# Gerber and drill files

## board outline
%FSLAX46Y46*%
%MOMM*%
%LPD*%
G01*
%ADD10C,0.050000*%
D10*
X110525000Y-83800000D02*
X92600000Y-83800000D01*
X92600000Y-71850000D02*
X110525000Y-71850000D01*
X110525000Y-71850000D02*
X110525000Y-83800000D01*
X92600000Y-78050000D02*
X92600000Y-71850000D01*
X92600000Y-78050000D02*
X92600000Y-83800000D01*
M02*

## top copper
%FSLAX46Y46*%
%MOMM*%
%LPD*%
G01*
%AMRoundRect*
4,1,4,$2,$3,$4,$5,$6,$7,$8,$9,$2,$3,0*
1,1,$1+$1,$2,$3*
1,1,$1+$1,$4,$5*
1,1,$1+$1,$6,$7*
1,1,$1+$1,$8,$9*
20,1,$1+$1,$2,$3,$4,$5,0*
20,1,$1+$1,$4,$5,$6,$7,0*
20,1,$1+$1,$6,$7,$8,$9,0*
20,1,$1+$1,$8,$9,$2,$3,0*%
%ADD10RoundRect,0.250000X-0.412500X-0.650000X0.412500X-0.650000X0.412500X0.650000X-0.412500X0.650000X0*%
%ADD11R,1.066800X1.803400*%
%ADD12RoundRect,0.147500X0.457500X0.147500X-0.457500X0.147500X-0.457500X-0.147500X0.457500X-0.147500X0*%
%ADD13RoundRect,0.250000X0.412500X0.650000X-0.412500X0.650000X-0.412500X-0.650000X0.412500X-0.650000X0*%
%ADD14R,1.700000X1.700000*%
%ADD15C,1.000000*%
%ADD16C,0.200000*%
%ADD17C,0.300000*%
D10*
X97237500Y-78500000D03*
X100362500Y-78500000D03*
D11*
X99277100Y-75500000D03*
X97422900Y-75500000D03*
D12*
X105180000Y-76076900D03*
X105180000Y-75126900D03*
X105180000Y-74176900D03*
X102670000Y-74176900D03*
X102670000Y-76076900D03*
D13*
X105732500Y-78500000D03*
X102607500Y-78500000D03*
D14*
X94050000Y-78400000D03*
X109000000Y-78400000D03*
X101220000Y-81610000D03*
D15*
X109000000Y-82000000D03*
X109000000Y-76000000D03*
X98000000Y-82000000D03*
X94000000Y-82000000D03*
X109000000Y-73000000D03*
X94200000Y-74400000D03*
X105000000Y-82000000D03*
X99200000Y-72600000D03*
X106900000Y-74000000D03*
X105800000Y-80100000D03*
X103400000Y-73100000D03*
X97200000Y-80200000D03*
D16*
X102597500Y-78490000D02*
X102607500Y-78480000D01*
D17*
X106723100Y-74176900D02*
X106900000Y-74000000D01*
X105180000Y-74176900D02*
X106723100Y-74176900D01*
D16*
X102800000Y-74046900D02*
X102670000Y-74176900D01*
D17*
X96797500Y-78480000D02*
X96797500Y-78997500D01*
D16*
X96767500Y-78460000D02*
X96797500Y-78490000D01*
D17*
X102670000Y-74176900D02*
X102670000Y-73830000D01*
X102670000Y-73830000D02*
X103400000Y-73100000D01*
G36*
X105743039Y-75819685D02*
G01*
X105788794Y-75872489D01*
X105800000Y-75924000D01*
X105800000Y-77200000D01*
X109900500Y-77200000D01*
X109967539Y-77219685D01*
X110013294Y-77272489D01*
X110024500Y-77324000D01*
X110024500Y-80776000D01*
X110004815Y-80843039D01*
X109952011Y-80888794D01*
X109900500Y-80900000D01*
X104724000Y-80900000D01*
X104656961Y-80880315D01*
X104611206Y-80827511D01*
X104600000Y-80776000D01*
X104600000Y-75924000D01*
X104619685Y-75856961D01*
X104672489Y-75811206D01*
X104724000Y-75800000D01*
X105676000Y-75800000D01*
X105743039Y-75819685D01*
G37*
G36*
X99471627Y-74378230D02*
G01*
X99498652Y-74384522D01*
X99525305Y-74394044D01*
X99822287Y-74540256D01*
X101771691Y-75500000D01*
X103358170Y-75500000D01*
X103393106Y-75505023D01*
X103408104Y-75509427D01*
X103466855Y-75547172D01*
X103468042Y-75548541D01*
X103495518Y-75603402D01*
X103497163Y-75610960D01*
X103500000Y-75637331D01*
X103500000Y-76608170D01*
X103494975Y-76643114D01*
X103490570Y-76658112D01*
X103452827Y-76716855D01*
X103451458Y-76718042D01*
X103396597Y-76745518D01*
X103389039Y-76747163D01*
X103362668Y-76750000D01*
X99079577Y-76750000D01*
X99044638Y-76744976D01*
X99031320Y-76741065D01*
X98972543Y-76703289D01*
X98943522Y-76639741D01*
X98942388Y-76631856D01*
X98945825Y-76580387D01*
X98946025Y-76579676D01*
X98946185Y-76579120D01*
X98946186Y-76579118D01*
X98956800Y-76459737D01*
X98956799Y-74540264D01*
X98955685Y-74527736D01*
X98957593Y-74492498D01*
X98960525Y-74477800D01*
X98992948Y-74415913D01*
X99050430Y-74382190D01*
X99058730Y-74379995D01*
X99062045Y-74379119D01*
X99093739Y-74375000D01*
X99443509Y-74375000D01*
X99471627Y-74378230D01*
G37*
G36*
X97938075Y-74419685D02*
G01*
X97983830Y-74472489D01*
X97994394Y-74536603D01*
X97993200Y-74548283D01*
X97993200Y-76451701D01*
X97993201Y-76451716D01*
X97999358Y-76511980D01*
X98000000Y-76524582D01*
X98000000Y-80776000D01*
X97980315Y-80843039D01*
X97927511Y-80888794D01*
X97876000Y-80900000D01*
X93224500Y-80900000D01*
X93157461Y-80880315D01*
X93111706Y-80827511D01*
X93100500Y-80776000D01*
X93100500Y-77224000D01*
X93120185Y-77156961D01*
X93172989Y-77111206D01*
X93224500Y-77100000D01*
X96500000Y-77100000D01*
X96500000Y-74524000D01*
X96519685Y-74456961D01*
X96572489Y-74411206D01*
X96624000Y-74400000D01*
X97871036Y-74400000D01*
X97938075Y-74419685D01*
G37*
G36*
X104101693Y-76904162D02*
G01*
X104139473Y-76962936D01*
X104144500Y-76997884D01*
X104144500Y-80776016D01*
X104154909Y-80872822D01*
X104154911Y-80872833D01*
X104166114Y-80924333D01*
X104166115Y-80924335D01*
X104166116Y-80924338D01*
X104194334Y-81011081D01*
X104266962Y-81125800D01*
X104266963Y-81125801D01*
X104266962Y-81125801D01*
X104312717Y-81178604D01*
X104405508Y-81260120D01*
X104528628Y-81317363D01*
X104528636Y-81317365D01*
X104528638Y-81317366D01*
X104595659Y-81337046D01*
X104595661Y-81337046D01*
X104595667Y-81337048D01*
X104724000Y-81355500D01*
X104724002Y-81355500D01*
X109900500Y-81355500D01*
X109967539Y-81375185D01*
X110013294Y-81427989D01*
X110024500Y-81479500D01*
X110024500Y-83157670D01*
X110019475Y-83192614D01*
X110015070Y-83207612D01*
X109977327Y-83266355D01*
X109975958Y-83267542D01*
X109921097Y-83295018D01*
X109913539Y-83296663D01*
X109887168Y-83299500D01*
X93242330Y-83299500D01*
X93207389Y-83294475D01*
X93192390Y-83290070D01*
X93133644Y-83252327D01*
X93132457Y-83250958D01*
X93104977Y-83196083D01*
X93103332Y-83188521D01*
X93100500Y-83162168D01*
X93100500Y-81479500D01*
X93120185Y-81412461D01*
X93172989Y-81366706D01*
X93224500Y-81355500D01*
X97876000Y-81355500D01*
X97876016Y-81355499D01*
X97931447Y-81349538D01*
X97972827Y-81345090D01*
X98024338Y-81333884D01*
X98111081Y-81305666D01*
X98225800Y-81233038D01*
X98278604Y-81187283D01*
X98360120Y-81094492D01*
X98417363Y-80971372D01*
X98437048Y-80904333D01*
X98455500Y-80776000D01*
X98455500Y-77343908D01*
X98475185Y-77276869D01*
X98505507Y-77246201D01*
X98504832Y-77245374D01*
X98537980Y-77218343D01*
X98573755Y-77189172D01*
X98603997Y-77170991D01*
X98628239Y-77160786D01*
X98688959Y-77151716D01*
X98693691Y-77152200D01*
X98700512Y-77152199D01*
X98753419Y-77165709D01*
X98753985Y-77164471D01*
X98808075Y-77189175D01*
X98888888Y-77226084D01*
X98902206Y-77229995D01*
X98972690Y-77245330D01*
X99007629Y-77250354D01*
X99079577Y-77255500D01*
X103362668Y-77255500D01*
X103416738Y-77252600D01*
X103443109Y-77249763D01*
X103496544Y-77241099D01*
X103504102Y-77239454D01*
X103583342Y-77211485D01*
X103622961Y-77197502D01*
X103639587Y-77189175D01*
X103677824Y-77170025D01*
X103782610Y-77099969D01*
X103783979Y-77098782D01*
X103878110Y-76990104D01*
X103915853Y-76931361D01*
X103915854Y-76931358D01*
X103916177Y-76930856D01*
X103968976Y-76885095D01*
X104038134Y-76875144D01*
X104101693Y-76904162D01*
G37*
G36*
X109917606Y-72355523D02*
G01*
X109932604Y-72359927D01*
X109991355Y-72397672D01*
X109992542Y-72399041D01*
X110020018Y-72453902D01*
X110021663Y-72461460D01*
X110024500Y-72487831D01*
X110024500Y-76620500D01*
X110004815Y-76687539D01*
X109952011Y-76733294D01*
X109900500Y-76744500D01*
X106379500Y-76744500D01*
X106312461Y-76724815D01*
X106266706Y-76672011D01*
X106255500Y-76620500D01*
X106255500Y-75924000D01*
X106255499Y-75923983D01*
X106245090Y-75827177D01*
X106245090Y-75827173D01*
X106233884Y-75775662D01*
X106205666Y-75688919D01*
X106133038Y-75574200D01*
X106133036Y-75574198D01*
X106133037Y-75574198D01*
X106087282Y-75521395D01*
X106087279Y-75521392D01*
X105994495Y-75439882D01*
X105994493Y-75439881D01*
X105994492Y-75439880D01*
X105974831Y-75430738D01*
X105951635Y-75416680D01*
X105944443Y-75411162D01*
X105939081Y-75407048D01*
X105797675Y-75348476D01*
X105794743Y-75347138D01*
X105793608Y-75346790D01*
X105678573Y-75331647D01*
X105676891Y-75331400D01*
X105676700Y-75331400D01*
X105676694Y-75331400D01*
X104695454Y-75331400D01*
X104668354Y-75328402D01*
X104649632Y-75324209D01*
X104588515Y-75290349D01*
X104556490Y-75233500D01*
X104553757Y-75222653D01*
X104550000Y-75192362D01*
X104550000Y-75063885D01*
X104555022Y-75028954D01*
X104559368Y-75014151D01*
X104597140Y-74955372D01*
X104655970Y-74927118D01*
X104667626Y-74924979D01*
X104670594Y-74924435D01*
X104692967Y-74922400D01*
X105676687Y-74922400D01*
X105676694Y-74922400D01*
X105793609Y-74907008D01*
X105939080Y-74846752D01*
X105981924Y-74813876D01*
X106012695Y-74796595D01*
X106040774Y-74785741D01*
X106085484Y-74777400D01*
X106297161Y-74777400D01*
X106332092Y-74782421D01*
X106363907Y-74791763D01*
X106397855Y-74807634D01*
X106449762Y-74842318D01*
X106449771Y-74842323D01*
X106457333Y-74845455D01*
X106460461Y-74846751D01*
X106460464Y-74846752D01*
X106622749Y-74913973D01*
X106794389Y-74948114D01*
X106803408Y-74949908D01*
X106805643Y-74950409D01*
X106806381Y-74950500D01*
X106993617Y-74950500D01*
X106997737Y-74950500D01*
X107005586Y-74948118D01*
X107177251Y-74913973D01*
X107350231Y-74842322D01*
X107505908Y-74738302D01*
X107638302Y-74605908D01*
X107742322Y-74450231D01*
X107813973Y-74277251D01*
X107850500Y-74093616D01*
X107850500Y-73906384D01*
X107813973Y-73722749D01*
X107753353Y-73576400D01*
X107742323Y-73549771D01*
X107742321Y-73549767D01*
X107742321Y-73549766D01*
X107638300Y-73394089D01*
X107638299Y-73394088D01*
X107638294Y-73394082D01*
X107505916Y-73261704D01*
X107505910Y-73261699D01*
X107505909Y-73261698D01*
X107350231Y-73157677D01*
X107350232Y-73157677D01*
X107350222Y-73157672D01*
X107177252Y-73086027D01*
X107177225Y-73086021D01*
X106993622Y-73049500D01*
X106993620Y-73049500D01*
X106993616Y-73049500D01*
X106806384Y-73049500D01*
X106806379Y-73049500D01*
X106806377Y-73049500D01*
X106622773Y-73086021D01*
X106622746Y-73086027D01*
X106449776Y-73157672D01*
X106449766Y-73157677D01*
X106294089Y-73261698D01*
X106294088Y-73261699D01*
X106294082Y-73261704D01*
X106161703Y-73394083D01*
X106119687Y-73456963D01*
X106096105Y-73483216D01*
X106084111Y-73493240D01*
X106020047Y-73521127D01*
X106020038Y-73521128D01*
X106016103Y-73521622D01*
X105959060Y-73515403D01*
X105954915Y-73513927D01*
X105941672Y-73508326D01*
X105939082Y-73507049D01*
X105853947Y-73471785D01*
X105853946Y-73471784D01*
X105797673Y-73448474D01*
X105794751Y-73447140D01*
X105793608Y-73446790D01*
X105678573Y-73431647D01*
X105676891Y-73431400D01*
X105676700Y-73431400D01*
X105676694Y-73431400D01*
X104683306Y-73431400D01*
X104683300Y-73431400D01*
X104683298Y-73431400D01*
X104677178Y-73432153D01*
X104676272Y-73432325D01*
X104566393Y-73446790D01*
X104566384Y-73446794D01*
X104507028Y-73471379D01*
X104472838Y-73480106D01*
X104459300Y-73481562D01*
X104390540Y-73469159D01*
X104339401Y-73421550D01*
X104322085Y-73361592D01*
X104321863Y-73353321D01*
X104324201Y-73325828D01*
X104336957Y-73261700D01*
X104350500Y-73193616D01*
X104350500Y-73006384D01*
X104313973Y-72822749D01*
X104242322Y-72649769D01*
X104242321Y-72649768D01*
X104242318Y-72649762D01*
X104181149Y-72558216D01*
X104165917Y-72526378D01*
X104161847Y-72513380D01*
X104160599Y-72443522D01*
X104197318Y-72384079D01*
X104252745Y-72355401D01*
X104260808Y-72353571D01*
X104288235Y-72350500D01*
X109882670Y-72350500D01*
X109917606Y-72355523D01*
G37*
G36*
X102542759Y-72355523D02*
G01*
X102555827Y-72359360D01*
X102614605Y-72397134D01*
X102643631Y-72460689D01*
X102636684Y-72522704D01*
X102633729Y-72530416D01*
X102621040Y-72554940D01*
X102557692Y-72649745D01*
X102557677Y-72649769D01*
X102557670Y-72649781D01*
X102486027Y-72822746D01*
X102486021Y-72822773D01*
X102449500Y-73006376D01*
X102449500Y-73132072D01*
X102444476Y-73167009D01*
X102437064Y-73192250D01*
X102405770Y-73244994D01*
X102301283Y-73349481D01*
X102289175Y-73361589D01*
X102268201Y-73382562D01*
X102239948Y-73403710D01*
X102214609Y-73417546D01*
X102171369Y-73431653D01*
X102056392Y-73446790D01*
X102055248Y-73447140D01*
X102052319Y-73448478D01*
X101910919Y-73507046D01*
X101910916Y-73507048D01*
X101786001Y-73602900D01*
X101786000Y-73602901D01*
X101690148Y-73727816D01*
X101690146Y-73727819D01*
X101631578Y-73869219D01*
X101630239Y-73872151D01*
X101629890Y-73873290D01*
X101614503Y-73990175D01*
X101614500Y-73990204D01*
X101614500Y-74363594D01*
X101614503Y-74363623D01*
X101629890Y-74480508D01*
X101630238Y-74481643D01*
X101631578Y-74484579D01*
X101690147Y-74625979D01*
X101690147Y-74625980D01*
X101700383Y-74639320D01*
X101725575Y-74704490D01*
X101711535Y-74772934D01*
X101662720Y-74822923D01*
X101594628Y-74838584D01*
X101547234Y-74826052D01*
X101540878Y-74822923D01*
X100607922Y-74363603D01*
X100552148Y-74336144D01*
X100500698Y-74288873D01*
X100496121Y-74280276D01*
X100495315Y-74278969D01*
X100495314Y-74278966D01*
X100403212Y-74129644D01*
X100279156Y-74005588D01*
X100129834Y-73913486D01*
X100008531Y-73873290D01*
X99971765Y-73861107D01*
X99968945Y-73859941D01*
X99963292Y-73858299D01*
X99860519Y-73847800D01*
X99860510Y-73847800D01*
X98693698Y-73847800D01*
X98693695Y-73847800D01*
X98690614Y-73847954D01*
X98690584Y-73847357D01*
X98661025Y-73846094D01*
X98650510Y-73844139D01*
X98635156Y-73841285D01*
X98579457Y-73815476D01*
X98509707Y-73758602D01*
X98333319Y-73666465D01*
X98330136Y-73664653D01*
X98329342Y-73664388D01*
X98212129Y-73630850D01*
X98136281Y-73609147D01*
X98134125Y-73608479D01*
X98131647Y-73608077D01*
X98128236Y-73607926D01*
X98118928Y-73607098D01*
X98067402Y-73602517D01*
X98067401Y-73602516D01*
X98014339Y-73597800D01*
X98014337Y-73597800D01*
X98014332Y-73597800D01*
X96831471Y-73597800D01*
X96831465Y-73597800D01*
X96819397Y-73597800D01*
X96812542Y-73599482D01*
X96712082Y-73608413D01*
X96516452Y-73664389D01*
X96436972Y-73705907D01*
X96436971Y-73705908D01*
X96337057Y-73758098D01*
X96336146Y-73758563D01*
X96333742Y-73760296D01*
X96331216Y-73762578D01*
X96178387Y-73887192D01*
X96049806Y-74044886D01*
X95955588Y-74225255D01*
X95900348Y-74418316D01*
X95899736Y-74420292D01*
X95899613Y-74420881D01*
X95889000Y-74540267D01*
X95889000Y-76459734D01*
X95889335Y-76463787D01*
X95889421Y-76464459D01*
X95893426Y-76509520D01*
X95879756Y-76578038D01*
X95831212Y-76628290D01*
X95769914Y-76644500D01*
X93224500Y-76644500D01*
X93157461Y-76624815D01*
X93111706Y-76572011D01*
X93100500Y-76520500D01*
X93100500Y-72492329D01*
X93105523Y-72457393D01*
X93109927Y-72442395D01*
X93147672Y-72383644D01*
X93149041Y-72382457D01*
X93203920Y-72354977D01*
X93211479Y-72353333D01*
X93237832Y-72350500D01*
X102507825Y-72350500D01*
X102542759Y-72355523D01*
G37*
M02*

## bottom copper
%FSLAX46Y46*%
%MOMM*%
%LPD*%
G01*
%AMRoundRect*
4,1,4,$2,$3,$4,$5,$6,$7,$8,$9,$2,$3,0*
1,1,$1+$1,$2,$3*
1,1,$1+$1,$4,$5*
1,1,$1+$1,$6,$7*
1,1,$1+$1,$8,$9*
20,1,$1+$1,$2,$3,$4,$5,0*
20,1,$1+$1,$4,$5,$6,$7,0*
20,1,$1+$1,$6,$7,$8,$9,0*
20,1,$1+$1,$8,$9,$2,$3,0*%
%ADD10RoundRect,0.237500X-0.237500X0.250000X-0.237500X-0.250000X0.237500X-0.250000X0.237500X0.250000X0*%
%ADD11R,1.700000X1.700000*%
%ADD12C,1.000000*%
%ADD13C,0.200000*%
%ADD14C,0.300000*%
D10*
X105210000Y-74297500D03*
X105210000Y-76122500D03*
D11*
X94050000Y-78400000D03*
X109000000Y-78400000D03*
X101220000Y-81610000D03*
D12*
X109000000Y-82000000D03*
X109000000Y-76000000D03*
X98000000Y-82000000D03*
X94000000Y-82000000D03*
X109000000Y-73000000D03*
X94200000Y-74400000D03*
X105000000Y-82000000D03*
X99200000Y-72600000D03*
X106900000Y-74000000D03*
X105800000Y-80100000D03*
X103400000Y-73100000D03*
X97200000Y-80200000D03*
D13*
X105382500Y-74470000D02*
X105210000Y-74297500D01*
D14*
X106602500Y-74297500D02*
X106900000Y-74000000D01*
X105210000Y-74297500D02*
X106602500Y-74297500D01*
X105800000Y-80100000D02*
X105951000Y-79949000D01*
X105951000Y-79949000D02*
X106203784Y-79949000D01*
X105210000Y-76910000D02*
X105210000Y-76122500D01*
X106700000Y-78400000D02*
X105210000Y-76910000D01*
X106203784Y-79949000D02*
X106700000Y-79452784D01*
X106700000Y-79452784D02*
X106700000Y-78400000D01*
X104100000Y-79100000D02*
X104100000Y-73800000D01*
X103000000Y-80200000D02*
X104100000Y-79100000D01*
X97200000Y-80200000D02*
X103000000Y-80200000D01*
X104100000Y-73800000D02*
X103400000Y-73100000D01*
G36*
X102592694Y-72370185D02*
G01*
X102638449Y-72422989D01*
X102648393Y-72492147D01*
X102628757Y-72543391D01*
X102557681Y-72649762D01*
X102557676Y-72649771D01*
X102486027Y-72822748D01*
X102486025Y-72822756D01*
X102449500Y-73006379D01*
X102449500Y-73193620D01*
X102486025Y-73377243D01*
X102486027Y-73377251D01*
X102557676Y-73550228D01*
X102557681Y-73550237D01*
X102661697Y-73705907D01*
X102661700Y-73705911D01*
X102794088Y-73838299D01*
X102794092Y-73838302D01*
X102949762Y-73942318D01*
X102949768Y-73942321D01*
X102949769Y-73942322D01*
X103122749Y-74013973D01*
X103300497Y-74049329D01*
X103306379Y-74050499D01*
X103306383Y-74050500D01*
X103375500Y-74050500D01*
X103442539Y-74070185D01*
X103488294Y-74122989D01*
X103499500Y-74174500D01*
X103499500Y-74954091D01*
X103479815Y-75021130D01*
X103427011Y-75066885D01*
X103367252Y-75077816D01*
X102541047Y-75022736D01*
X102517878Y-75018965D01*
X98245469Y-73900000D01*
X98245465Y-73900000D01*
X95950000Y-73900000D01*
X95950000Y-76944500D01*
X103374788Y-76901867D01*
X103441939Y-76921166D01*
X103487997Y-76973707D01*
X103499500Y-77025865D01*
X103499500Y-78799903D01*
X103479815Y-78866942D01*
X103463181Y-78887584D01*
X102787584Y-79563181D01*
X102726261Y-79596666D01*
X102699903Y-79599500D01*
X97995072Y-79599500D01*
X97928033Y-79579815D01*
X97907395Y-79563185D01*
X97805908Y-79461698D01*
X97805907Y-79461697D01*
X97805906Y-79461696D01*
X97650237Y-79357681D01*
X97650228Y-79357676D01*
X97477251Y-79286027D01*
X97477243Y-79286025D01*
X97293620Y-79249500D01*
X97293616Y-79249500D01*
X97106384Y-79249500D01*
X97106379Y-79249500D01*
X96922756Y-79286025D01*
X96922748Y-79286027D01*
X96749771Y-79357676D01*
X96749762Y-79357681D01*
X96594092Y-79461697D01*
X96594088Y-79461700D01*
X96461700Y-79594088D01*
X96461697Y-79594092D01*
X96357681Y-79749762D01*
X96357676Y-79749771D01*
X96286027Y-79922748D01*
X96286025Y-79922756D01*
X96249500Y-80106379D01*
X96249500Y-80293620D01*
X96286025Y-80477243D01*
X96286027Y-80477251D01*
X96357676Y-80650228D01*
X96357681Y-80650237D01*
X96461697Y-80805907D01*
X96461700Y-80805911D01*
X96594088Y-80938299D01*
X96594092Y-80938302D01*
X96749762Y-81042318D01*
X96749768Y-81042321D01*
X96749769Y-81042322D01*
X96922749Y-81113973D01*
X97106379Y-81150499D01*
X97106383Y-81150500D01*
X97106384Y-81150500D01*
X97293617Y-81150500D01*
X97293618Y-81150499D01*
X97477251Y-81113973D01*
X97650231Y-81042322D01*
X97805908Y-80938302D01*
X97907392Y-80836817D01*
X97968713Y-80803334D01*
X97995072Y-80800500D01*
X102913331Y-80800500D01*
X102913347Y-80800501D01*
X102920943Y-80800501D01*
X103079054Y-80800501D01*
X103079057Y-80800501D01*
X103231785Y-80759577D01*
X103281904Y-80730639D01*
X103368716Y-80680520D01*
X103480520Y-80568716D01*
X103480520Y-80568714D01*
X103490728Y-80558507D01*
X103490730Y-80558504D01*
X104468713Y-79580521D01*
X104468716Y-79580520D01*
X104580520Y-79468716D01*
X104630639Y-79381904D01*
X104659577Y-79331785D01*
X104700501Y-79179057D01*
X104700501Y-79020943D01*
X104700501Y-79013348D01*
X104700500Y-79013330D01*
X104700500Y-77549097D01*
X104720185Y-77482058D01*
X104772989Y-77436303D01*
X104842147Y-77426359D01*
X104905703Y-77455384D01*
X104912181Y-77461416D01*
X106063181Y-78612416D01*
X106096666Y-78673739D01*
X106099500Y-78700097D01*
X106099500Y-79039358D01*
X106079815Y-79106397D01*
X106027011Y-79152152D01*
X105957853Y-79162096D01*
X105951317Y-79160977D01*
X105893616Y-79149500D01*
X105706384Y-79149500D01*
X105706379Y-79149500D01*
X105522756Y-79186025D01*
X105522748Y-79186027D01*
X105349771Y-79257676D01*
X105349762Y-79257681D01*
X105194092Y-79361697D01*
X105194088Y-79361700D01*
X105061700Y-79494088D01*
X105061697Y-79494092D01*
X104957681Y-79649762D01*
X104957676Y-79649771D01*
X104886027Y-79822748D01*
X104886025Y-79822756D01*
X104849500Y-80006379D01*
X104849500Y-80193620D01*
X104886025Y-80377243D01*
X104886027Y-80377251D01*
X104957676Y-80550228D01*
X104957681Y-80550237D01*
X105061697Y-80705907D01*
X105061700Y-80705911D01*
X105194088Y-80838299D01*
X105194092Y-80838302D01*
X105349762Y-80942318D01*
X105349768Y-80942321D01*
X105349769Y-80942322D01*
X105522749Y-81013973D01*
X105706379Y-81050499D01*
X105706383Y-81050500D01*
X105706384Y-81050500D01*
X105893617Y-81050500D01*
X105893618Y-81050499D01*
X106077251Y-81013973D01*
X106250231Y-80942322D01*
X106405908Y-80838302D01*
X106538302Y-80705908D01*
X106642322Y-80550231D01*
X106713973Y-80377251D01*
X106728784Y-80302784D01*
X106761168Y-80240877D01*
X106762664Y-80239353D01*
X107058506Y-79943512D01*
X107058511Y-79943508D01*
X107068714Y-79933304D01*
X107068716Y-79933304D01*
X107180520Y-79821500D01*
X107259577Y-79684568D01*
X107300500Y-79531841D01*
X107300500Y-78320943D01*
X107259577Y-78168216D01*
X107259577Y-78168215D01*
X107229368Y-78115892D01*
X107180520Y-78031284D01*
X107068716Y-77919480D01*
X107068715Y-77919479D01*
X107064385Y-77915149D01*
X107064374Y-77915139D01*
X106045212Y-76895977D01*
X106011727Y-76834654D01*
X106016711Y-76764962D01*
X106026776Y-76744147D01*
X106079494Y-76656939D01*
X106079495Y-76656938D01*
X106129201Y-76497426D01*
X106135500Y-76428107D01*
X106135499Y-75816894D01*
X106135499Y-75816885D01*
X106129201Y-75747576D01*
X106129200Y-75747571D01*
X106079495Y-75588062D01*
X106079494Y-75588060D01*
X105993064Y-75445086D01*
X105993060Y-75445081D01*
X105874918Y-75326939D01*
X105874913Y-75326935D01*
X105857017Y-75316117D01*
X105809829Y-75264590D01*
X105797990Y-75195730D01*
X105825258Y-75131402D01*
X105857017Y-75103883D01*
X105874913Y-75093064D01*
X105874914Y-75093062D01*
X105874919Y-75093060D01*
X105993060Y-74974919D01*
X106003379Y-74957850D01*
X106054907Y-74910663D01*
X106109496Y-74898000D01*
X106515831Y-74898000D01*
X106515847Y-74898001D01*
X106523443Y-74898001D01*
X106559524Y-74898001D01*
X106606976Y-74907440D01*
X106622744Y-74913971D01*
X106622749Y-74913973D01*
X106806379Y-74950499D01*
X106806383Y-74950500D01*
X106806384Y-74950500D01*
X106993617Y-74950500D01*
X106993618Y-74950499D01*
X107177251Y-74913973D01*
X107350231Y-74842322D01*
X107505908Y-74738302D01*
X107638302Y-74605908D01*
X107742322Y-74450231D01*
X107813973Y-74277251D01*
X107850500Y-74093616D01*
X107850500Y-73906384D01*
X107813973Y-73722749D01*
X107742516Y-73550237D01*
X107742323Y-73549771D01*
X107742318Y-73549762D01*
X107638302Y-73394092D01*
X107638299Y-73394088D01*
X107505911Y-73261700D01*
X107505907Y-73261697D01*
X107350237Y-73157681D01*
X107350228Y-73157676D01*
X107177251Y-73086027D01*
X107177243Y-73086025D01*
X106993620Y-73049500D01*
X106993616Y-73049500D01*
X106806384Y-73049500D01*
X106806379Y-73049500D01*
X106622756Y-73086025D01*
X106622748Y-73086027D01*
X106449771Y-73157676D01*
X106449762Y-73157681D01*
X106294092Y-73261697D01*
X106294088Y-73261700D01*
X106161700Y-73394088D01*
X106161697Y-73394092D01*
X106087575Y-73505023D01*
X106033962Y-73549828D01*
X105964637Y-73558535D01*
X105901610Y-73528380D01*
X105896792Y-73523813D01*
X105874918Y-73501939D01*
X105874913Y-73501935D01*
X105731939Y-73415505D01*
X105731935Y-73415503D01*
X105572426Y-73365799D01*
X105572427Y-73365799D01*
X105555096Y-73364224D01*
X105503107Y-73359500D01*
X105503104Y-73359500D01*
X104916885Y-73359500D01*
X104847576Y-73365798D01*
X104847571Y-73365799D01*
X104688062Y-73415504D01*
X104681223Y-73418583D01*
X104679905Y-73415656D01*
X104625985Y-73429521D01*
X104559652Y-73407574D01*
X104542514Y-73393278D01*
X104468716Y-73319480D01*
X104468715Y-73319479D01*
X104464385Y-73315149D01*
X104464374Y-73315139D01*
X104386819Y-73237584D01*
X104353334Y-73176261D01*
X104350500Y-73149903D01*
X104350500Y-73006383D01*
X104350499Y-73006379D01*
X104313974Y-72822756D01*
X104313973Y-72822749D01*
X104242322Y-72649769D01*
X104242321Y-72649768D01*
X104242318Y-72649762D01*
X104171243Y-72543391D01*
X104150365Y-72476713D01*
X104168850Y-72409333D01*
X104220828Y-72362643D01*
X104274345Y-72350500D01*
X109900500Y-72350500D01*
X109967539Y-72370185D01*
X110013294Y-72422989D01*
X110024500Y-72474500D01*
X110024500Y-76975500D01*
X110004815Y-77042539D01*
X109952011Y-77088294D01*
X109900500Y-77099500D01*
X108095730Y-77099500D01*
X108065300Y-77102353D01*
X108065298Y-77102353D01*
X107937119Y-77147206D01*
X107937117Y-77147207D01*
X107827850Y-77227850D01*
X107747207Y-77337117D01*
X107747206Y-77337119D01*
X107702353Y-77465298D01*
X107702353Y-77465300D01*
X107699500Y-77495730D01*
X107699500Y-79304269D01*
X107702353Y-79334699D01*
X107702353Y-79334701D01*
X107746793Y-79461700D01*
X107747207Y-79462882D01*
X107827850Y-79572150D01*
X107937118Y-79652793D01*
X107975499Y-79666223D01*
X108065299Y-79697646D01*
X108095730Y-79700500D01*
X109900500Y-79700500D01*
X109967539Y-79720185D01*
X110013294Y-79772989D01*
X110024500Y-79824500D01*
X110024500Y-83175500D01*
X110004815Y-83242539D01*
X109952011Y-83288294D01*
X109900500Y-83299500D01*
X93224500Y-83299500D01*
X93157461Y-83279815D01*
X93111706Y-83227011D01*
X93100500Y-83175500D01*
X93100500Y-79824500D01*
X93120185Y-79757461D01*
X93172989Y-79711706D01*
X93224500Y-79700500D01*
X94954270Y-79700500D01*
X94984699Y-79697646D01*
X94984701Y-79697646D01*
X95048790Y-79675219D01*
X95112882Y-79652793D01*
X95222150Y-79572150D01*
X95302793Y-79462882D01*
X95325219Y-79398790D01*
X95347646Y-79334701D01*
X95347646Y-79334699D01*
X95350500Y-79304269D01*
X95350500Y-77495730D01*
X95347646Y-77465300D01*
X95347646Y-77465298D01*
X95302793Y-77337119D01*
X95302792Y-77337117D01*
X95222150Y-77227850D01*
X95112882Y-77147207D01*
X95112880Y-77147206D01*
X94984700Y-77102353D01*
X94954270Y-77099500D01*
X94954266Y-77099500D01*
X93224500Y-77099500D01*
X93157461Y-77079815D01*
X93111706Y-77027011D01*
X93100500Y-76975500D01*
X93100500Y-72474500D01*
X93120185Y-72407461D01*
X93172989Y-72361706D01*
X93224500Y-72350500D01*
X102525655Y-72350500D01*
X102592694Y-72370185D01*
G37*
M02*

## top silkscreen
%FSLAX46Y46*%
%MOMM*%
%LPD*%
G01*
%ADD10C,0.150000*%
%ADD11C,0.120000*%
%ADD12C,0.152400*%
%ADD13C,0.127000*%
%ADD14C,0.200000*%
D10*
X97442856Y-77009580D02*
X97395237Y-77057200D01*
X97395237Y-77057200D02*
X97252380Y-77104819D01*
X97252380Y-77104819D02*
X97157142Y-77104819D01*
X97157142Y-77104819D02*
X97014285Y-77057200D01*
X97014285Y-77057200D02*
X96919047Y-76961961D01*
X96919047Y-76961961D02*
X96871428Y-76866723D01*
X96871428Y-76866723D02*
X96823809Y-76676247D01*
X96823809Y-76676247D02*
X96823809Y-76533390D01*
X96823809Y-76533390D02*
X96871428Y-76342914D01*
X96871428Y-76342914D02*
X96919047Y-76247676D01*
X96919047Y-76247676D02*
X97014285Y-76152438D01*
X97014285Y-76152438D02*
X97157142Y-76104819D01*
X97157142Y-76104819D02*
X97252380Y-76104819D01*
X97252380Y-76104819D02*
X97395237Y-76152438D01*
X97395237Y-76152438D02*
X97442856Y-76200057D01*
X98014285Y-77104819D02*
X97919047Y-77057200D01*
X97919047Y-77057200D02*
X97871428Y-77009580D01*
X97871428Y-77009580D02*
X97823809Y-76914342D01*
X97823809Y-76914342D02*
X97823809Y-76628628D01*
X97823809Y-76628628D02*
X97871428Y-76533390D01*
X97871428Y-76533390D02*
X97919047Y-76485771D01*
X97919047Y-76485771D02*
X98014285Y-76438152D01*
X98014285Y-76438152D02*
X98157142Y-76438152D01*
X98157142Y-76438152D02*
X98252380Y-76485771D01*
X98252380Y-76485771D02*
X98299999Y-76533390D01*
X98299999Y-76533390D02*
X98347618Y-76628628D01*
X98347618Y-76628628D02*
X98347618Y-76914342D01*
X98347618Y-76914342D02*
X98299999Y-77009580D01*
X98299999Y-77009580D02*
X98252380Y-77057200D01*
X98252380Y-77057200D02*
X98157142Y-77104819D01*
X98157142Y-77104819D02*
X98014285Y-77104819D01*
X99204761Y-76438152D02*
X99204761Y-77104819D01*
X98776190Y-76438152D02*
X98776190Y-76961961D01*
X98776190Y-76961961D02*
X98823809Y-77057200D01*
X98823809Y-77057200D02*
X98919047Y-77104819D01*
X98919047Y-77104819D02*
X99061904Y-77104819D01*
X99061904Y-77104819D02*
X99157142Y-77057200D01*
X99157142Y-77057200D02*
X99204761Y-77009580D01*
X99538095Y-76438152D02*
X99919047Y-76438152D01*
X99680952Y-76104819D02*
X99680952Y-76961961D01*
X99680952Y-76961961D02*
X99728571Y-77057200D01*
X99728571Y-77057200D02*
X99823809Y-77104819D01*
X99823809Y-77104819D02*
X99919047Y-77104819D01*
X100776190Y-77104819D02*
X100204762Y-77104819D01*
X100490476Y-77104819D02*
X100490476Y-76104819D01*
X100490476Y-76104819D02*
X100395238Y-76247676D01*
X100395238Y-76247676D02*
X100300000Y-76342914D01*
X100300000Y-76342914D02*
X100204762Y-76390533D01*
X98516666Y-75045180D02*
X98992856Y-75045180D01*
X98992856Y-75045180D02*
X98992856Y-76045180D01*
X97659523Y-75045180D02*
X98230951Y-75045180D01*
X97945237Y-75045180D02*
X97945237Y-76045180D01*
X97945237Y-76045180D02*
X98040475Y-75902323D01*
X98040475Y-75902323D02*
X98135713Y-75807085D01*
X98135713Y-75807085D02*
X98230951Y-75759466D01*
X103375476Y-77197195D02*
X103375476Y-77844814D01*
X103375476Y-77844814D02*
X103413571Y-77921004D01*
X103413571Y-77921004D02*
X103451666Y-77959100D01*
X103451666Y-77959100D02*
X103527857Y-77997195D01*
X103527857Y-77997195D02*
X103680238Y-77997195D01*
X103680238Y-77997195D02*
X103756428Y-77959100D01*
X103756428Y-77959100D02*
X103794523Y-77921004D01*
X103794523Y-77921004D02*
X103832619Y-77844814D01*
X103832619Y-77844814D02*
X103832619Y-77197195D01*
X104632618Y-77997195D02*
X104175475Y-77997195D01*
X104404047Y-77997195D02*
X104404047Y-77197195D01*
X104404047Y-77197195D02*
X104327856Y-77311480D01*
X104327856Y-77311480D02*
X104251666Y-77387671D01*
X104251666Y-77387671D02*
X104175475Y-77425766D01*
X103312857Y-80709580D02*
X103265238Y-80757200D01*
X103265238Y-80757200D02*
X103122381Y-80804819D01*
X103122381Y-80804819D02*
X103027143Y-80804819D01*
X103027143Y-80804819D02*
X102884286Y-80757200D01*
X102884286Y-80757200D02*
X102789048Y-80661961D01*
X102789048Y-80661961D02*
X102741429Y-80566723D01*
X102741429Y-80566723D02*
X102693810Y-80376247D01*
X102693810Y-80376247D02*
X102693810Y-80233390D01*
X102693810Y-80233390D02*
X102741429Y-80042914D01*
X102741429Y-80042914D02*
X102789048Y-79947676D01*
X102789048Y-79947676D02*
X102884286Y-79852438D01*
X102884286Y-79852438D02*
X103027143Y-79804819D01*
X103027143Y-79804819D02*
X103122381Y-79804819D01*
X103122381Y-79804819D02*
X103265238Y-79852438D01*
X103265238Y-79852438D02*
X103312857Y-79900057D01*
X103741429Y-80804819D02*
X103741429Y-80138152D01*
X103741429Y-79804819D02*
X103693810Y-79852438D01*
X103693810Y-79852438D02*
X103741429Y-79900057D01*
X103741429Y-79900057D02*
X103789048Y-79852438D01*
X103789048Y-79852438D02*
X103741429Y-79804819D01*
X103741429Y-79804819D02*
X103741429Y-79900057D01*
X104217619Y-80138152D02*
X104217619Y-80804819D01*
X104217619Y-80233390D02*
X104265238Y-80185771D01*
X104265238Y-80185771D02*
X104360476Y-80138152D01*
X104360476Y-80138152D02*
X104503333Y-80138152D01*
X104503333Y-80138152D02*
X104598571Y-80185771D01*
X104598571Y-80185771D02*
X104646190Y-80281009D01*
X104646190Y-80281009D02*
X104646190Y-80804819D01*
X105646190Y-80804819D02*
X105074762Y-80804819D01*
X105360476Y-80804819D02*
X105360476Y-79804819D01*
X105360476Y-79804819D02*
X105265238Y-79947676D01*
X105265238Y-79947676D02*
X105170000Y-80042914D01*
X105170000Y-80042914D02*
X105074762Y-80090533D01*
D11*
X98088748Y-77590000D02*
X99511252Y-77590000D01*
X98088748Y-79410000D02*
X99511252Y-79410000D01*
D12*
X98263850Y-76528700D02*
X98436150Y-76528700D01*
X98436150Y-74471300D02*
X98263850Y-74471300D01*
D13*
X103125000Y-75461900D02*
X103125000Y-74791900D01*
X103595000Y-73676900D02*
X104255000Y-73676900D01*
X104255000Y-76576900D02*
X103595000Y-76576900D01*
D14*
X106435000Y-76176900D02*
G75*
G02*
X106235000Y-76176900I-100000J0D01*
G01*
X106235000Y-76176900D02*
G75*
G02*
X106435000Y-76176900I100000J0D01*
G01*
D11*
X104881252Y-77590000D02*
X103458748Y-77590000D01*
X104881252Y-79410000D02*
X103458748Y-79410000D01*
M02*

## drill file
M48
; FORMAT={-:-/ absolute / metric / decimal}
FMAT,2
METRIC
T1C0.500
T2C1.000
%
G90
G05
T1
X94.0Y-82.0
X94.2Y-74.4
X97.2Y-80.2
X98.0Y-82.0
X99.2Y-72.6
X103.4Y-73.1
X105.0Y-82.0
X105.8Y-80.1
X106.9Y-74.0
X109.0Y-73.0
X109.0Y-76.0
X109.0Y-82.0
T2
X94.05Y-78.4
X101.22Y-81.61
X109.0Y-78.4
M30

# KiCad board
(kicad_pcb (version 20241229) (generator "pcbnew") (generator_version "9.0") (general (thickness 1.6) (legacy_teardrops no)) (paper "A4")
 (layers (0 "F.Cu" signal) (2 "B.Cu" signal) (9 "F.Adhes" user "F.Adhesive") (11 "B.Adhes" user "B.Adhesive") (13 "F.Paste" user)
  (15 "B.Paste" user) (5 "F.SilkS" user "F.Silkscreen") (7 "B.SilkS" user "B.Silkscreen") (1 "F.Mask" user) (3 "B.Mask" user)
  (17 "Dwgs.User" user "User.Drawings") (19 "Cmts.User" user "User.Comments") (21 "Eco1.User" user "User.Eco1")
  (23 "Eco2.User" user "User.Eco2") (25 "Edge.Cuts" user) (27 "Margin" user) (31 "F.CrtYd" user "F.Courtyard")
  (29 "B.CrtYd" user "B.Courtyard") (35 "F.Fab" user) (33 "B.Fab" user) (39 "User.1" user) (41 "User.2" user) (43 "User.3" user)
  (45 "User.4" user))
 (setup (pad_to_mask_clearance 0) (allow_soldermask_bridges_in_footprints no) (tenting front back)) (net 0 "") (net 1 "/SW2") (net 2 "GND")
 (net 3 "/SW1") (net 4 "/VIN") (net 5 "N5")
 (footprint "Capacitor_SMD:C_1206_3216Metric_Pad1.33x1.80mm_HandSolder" (layer "F.Cu") (at 98.8 78.5)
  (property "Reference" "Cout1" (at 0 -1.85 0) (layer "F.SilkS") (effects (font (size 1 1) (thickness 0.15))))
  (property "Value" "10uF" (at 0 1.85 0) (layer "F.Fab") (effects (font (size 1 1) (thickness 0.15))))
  (fp_line (start -0.711252 -0.91) (end 0.711252 -0.91) (stroke (width 0.12) (type solid)) (layer "F.SilkS"))
  (fp_line (start -0.711252 0.91) (end 0.711252 0.91) (stroke (width 0.12) (type solid)) (layer "F.SilkS"))
  (pad "1" smd roundrect (at -1.5625 0) (size 1.325 1.8) (layers "F.Cu" "F.Mask" "F.Paste") (roundrect_rratio 0.188679) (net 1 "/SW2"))
  (pad "2" smd roundrect (at 1.5625 0) (size 1.325 1.8) (layers "F.Cu" "F.Mask" "F.Paste") (roundrect_rratio 0.188679) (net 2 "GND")))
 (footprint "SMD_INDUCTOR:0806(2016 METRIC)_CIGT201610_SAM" (layer "F.Cu") (at 98.35 75.5 180)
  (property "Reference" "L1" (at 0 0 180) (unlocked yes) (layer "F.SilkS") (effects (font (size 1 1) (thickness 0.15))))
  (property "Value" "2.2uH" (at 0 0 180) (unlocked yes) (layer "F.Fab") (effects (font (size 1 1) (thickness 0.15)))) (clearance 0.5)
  (fp_line (start 0.08615 -1.0287) (end -0.08615 -1.0287) (stroke (width 0.1524) (type solid)) (layer "F.SilkS"))
  (fp_line (start -0.08615 1.0287) (end 0.08615 1.0287) (stroke (width 0.1524) (type solid)) (layer "F.SilkS"))
  (pad "1" smd rect (at -0.9271 0 180) (size 1.0668 1.8034) (layers "F.Cu" "F.Mask" "F.Paste") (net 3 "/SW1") (clearance 0.75))
  (pad "2" smd rect (at 0.9271 0 180) (size 1.0668 1.8034) (layers "F.Cu" "F.Mask" "F.Paste") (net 1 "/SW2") (clearance 1))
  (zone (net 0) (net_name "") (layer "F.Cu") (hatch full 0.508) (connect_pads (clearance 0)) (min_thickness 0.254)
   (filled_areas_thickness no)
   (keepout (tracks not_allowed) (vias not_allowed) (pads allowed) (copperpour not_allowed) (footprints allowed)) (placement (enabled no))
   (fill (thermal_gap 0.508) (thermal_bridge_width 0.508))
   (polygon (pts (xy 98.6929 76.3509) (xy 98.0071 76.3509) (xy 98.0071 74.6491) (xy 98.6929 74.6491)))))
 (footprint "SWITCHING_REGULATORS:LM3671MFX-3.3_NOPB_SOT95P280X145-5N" (layer "F.Cu") (at 103.925 75.1269 180)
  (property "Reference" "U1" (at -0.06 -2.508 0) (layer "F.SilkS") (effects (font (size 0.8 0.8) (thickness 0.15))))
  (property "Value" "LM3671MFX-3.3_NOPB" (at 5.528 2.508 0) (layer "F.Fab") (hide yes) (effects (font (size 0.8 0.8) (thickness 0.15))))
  (fp_line (start 0.8 -0.335) (end 0.8 0.335) (stroke (width 0.127) (type solid)) (layer "F.SilkS"))
  (fp_line (start 0.33 1.45) (end -0.33 1.45) (stroke (width 0.127) (type solid)) (layer "F.SilkS"))
  (fp_line (start -0.33 -1.45) (end 0.33 -1.45) (stroke (width 0.127) (type solid)) (layer "F.SilkS"))
  (fp_circle (center -2.41 -1.05) (end -2.31 -1.05) (stroke (width 0.2) (type solid)) (fill no) (layer "F.SilkS"))
  (pad "1" smd roundrect (at -1.255 -0.95 180) (size 1.21 0.59) (layers "F.Cu" "F.Mask" "F.Paste") (roundrect_rratio 0.25) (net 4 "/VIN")
   (solder_mask_margin 0.102))
  (pad "2" smd roundrect (at -1.255 0 180) (size 1.21 0.59) (layers "F.Cu" "F.Mask" "F.Paste") (roundrect_rratio 0.25) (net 2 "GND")
   (solder_mask_margin 0.102))
  (pad "3" smd roundrect (at -1.255 0.95 180) (size 1.21 0.59) (layers "F.Cu" "F.Mask" "F.Paste") (roundrect_rratio 0.25) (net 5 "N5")
   (solder_mask_margin 0.102))
  (pad "4" smd roundrect (at 1.255 0.95 180) (size 1.21 0.59) (layers "F.Cu" "F.Mask" "F.Paste") (roundrect_rratio 0.25) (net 1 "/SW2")
   (solder_mask_margin 0.102))
  (pad "5" smd roundrect (at 1.255 -0.95 180) (size 1.21 0.59) (layers "F.Cu" "F.Mask" "F.Paste") (roundrect_rratio 0.25) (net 3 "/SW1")
   (solder_mask_margin 0.102)))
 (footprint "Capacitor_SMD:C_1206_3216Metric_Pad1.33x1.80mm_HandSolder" (layer "F.Cu") (at 104.17 78.5 180)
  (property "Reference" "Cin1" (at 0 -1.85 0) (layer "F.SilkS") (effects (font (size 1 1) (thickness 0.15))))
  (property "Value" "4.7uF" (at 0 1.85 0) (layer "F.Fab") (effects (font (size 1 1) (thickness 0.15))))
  (fp_line (start -0.711252 0.91) (end 0.711252 0.91) (stroke (width 0.12) (type solid)) (layer "F.SilkS"))
  (fp_line (start -0.711252 -0.91) (end 0.711252 -0.91) (stroke (width 0.12) (type solid)) (layer "F.SilkS"))
  (pad "1" smd roundrect (at -1.5625 0 180) (size 1.325 1.8) (layers "F.Cu" "F.Mask" "F.Paste") (roundrect_rratio 0.188679) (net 4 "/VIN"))
  (pad "2" smd roundrect (at 1.5625 0 180) (size 1.325 1.8) (layers "F.Cu" "F.Mask" "F.Paste") (roundrect_rratio 0.188679) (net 2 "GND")))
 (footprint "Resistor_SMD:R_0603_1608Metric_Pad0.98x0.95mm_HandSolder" (layer "B.Cu") (at 105.21 75.21 -90)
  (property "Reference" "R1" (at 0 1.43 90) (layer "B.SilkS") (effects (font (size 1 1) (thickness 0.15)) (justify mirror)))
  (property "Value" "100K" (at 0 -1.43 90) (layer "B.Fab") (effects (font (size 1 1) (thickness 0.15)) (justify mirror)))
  (pad "1" smd roundrect (at -0.9125 0 270) (size 0.975 0.95) (layers "B.Cu" "B.Mask" "B.Paste") (roundrect_rratio 0.25) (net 5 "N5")
   (clearance 0.45))
  (pad "2" smd roundrect (at 0.9125 0 270) (size 0.975 0.95) (layers "B.Cu" "B.Mask" "B.Paste") (roundrect_rratio 0.25) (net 4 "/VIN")
   (clearance 0.45)))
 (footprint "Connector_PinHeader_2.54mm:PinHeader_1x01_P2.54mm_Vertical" (layer "B.Cu") (at 94.05 78.4 180)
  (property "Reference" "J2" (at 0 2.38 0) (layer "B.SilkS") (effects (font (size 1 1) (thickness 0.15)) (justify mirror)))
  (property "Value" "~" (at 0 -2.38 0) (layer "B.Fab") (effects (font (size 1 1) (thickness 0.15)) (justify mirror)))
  (pad "3" thru_hole rect (at 0 0 180) (size 1.7 1.7) (drill 1) (layers "*.Cu" "*.Mask") (remove_unused_layers no) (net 1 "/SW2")))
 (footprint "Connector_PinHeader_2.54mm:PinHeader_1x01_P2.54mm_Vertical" (layer "B.Cu") (at 109 78.4 180)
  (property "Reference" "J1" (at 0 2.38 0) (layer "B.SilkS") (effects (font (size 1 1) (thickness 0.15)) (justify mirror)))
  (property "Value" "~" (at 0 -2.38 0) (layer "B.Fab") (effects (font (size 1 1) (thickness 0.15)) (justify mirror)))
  (pad "1" thru_hole rect (at 0 0 180) (size 1.7 1.7) (drill 1) (layers "*.Cu" "*.Mask") (remove_unused_layers no) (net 4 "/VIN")))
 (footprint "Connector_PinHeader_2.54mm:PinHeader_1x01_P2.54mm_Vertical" (layer "B.Cu") (at 101.22 81.61 180)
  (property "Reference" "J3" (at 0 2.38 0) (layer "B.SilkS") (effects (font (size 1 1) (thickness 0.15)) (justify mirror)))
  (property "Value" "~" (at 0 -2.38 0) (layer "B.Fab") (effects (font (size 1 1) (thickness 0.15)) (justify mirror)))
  (pad "2" thru_hole rect (at 0 0 180) (size 1.7 1.7) (drill 1) (layers "*.Cu" "*.Mask") (remove_unused_layers no) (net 2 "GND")))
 (gr_line (start 110.525 83.8) (end 92.6 83.8) (stroke (width 0.05) (type default)) (layer "Edge.Cuts"))
 (gr_line (start 92.6 71.85) (end 110.525 71.85) (stroke (width 0.05) (type default)) (layer "Edge.Cuts"))
 (gr_line (start 110.525 71.85) (end 110.525 83.8) (stroke (width 0.05) (type default)) (layer "Edge.Cuts"))
 (gr_line (start 92.6 78.05) (end 92.6 71.85) (stroke (width 0.05) (type default)) (layer "Edge.Cuts"))
 (gr_line (start 92.6 78.05) (end 92.6 83.8) (stroke (width 0.05) (type default)) (layer "Edge.Cuts"))
 (segment (start 102.5975 78.49) (end 102.6075 78.48) (width 0.2) (layer "F.Cu") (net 2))
 (via (at 109 82) (size 1) (drill 0.5) (layers "F.Cu" "B.Cu") (free yes) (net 2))
 (via (at 109 76) (size 1) (drill 0.5) (layers "F.Cu" "B.Cu") (free yes) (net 2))
 (via (at 98 82) (size 1) (drill 0.5) (layers "F.Cu" "B.Cu") (free yes) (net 2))
 (via (at 94 82) (size 1) (drill 0.5) (layers "F.Cu" "B.Cu") (free yes) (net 2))
 (via (at 109 73) (size 1) (drill 0.5) (layers "F.Cu" "B.Cu") (free yes) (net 2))
 (via (at 94.2 74.4) (size 1) (drill 0.5) (layers "F.Cu" "B.Cu") (free yes) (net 2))
 (via (at 105 82) (size 1) (drill 0.5) (layers "F.Cu" "B.Cu") (free yes) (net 2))
 (via (at 99.2 72.6) (size 1) (drill 0.5) (layers "F.Cu" "B.Cu") (free yes) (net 2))
 (segment (start 106.7231 74.1769) (end 106.9 74) (width 0.3) (layer "F.Cu") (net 5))
 (segment (start 105.18 74.1769) (end 106.7231 74.1769) (width 0.3) (layer "F.Cu") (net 5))
 (via (at 106.9 74) (size 1) (drill 0.5) (layers "F.Cu" "B.Cu") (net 5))
 (segment (start 105.3825 74.47) (end 105.21 74.2975) (width 0.2) (layer "B.Cu") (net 5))
 (segment (start 106.6025 74.2975) (end 106.9 74) (width 0.3) (layer "B.Cu") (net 5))
 (segment (start 105.21 74.2975) (end 106.6025 74.2975) (width 0.3) (layer "B.Cu") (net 5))
 (via (at 105.8 80.1) (size 1) (drill 0.5) (layers "F.Cu" "B.Cu") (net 4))
 (segment (start 105.8 80.1) (end 105.951 79.949) (width 0.3) (layer "B.Cu") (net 4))
 (segment (start 105.951 79.949) (end 106.203784 79.949) (width 0.3) (layer "B.Cu") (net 4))
 (segment (start 105.21 76.91) (end 105.21 76.1225) (width 0.3) (layer "B.Cu") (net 4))
 (segment (start 106.7 78.4) (end 105.21 76.91) (width 0.3) (layer "B.Cu") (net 4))
 (segment (start 106.203784 79.949) (end 106.7 79.452784) (width 0.3) (layer "B.Cu") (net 4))
 (segment (start 106.7 79.452784) (end 106.7 78.4) (width 0.3) (layer "B.Cu") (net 4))
 (segment (start 102.8 74.0469) (end 102.67 74.1769) (width 0.2) (layer "F.Cu") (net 1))
 (segment (start 96.7975 78.48) (end 96.7975 78.9975) (width 0.3) (layer "F.Cu") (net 1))
 (segment (start 96.7675 78.46) (end 96.7975 78.49) (width 0.2) (layer "F.Cu") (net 1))
 (segment (start 102.67 74.1769) (end 102.67 73.83) (width 0.3) (layer "F.Cu") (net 1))
 (segment (start 102.67 73.83) (end 103.4 73.1) (width 0.3) (layer "F.Cu") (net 1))
 (via (at 103.4 73.1) (size 1) (drill 0.5) (layers "F.Cu" "B.Cu") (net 1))
 (via (at 97.2 80.2) (size 1) (drill 0.5) (layers "F.Cu" "B.Cu") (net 1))
 (segment (start 104.1 79.1) (end 104.1 73.8) (width 0.3) (layer "B.Cu") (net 1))
 (segment (start 103 80.2) (end 104.1 79.1) (width 0.3) (layer "B.Cu") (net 1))
 (segment (start 97.2 80.2) (end 103 80.2) (width 0.3) (layer "B.Cu") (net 1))
 (segment (start 104.1 73.8) (end 103.4 73.1) (width 0.3) (layer "B.Cu") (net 1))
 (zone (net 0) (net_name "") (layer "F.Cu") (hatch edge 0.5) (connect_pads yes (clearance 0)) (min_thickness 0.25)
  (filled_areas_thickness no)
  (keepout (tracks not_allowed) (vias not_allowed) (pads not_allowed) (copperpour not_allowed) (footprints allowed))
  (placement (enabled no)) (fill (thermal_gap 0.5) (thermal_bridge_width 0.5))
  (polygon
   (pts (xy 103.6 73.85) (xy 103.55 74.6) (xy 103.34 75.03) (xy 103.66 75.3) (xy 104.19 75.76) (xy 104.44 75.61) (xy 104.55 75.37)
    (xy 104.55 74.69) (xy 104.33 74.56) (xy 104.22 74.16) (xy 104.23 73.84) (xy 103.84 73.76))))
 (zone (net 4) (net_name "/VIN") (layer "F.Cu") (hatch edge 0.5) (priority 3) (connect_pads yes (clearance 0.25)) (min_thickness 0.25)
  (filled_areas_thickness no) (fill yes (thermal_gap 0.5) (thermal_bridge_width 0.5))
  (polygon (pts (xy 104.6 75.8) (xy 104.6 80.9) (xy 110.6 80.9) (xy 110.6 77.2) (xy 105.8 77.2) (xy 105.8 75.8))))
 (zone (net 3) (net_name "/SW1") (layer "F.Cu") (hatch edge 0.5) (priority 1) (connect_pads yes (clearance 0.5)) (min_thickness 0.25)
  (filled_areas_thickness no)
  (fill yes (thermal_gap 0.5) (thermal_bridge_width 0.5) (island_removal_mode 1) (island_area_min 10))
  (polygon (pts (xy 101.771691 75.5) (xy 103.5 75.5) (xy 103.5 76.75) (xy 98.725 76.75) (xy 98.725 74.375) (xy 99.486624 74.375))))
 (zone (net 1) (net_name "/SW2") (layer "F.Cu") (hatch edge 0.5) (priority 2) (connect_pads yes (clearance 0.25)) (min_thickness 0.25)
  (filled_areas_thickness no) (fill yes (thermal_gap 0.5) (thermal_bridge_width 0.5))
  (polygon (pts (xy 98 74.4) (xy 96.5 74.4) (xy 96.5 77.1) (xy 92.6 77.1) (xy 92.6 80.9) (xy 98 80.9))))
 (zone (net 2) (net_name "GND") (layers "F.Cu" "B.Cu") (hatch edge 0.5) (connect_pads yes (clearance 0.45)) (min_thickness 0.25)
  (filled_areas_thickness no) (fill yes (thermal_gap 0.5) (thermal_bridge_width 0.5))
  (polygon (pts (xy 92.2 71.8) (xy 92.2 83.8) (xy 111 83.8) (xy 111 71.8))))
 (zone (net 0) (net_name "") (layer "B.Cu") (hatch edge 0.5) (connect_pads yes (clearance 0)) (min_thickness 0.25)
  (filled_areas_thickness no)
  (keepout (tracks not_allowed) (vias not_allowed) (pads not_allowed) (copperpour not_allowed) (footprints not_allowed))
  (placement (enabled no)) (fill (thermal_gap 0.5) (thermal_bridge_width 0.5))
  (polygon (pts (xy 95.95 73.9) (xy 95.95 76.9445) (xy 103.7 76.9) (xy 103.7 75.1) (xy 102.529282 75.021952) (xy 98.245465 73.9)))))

